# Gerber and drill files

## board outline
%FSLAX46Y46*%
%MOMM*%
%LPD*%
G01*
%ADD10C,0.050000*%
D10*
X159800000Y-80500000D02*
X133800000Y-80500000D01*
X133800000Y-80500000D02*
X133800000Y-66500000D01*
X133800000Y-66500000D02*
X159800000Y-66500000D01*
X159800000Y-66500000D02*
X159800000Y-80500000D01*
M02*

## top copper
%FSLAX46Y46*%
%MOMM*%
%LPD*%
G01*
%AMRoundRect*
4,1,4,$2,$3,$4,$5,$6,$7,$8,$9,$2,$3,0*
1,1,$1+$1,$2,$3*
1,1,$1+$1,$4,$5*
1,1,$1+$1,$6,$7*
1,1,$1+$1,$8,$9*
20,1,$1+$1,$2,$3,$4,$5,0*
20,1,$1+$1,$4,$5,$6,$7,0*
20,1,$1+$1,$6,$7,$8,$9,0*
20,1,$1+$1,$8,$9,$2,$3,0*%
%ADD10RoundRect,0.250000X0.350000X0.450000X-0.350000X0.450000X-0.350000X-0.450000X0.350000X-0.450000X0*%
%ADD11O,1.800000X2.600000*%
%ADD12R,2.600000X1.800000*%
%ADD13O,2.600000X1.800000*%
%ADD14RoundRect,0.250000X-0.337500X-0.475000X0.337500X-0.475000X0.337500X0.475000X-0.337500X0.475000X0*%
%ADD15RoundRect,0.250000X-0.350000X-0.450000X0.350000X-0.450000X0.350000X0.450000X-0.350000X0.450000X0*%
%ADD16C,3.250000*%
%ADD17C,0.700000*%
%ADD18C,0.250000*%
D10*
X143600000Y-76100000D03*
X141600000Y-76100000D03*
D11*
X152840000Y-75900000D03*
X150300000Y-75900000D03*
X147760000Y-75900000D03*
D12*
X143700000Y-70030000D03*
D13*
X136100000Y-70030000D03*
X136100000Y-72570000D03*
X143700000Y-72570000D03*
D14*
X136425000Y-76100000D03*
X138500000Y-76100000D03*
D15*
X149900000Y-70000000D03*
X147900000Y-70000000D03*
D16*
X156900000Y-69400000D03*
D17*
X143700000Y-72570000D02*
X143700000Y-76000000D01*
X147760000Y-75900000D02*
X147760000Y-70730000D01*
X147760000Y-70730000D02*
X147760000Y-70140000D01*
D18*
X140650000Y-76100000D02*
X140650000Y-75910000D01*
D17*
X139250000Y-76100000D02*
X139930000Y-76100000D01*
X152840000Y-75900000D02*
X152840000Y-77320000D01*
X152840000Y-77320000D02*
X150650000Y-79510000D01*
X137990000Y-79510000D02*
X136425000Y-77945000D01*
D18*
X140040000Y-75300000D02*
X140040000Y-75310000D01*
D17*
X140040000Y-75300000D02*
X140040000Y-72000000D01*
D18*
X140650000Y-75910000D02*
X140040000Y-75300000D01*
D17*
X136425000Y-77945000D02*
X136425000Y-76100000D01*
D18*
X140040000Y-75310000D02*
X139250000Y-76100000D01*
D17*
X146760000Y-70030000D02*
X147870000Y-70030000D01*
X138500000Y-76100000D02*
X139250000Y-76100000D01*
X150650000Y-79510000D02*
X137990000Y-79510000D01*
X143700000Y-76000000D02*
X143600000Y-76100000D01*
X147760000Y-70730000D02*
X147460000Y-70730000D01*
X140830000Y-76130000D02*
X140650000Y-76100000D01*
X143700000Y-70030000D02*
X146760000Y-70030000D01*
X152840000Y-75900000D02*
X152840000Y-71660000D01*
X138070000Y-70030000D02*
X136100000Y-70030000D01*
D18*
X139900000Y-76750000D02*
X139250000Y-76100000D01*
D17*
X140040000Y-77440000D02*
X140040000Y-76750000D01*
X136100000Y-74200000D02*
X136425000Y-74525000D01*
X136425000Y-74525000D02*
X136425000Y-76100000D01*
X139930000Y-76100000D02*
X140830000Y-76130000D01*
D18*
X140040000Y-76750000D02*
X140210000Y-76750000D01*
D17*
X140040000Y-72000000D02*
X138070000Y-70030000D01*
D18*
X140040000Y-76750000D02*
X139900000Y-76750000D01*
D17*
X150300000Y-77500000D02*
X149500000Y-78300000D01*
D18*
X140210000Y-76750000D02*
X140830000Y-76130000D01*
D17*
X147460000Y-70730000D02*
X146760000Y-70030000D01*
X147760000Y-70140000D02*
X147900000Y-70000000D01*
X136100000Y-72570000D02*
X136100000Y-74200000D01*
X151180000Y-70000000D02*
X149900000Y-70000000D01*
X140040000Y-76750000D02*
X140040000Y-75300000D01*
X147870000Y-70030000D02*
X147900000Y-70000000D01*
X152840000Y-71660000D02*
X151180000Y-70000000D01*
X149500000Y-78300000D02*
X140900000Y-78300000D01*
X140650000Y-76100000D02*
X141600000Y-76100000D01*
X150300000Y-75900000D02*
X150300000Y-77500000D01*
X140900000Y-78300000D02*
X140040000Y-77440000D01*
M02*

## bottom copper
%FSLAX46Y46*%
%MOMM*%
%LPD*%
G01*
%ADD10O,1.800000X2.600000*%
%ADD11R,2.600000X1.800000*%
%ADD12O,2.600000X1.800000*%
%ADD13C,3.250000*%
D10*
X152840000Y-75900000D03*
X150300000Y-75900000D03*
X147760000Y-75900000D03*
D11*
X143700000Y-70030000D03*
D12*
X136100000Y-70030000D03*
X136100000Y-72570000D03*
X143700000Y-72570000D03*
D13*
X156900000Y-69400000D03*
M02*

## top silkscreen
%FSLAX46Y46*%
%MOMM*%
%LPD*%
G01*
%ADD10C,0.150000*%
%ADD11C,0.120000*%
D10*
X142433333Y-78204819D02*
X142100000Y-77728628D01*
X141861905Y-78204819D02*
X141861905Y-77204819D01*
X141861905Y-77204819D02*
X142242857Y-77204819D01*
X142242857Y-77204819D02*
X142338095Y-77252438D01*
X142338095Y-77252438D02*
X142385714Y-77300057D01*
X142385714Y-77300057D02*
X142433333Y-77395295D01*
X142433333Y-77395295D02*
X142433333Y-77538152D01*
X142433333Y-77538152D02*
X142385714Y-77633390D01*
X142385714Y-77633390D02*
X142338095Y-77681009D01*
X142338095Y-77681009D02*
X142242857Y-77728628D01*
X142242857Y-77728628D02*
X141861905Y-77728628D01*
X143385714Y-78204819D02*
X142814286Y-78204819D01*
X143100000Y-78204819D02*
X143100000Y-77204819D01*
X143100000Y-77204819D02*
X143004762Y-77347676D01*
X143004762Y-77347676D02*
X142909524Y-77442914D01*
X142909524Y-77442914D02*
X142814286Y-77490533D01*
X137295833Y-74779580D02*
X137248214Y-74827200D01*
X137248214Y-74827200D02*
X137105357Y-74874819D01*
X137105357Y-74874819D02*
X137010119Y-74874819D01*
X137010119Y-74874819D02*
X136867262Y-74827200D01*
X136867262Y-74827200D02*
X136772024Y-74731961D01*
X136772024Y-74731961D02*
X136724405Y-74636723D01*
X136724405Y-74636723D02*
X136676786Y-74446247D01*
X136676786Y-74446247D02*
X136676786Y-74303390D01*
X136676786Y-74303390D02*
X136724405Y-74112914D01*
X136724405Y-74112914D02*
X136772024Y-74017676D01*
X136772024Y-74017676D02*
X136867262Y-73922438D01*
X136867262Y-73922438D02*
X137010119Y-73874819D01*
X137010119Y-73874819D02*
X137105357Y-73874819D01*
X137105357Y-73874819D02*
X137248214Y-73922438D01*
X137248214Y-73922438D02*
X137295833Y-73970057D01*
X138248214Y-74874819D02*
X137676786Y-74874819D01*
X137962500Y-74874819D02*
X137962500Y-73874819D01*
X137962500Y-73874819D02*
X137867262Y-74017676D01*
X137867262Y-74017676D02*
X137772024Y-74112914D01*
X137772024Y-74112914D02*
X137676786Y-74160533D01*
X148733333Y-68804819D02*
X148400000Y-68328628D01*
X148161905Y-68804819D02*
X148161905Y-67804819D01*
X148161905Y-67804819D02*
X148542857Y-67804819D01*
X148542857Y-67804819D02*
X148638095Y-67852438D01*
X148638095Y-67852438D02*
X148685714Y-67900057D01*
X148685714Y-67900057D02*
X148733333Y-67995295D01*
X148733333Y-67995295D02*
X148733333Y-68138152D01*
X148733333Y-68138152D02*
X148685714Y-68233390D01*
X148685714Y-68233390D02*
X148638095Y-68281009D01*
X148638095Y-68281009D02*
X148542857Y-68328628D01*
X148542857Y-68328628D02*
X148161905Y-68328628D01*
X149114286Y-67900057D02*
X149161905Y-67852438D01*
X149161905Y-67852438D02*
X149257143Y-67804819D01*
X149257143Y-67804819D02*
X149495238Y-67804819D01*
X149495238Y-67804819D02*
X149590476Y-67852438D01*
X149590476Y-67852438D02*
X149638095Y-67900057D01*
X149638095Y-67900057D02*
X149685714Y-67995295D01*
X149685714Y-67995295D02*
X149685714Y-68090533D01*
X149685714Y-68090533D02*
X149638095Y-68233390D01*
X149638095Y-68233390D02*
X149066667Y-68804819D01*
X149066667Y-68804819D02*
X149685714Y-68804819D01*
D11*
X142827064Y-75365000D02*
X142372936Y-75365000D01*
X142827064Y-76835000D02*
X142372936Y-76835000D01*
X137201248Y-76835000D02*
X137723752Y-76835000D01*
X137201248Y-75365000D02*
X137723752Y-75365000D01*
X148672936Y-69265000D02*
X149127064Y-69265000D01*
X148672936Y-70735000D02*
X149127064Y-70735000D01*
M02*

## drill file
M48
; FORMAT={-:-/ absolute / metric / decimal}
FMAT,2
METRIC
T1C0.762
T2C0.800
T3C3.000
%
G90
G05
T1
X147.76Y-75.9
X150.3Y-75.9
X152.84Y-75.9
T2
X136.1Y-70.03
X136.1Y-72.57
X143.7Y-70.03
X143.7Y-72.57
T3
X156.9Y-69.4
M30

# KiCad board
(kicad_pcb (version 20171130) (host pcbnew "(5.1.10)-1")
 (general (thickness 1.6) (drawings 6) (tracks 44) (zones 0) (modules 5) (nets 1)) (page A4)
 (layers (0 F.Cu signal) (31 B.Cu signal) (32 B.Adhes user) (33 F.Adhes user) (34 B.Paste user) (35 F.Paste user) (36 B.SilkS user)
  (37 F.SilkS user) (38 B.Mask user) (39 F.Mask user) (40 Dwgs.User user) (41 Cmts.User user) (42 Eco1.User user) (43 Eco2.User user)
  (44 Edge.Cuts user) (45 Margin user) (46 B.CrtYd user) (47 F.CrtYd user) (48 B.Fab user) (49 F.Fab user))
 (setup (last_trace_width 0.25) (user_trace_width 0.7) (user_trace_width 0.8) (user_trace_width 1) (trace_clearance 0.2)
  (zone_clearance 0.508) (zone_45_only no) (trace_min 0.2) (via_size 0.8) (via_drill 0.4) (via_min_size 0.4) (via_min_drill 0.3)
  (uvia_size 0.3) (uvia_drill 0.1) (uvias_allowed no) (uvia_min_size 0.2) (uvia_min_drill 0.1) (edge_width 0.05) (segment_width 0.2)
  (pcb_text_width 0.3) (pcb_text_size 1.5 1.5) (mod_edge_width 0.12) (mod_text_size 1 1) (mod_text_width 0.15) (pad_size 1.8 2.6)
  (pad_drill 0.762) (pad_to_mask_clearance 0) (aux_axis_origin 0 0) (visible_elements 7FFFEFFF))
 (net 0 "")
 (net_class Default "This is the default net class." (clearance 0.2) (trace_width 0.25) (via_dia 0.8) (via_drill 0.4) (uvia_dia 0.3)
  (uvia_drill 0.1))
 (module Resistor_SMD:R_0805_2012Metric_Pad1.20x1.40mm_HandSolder (layer F.Cu) (at 142.6 76.1 180)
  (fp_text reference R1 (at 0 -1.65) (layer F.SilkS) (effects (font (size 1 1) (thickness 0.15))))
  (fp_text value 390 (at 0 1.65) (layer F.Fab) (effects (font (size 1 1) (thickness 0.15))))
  (fp_line (start -0.227064 0.735) (end 0.227064 0.735) (layer F.SilkS) (width 0.12))
  (fp_line (start -0.227064 -0.735) (end 0.227064 -0.735) (layer F.SilkS) (width 0.12))
  (pad 1 smd roundrect (at -1 0 180) (size 1.2 1.4) (layers F.Cu F.Paste F.Mask) (roundrect_rratio 0.208333))
  (pad 2 smd roundrect (at 1 0 180) (size 1.2 1.4) (layers F.Cu F.Paste F.Mask) (roundrect_rratio 0.208333)))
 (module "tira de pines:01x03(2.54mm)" (layer B.Cu) (at 150.3 73.36 180)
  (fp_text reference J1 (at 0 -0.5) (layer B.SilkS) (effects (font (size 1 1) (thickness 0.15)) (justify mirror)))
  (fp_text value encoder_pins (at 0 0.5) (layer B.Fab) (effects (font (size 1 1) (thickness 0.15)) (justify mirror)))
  (pad 1 thru_hole oval (at -2.54 -2.54 180) (size 1.8 2.6) (drill 0.762) (layers *.Cu *.Mask))
  (pad 2 thru_hole oval (at 0 -2.54 180) (size 1.8 2.6) (drill 0.762) (layers *.Cu *.Mask))
  (pad 3 thru_hole oval (at 2.54 -2.54 180) (size 1.8 2.6) (drill 0.762) (layers *.Cu *.Mask)))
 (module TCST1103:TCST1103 (layer B.Cu) (at 139.9 71.3 180)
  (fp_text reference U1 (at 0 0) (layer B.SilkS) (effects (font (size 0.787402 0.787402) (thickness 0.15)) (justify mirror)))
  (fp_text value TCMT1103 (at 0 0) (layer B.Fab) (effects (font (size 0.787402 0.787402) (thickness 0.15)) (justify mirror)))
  (pad 1 thru_hole rect (at -3.8 1.27 180) (size 2.6 1.8) (drill 0.8) (layers *.Cu *.Mask) (solder_mask_margin 0.102))
  (pad 3 thru_hole oval (at 3.8 1.27 180) (size 2.6 1.8) (drill 0.8) (layers *.Cu *.Mask) (solder_mask_margin 0.102))
  (pad 4 thru_hole oval (at 3.8 -1.27 180) (size 2.6 1.8) (drill 0.8) (layers *.Cu *.Mask) (solder_mask_margin 0.102))
  (pad 2 thru_hole oval (at -3.8 -1.27 180) (size 2.6 1.8) (drill 0.8) (layers *.Cu *.Mask) (solder_mask_margin 0.102)))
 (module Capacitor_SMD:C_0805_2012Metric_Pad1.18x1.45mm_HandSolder (layer F.Cu) (at 137.4625 76.1)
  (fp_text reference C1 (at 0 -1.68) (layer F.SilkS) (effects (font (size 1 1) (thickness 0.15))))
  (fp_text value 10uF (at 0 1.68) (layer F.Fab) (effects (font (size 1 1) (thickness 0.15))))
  (fp_line (start -0.261252 0.735) (end 0.261252 0.735) (layer F.SilkS) (width 0.12))
  (fp_line (start -0.261252 -0.735) (end 0.261252 -0.735) (layer F.SilkS) (width 0.12))
  (pad 1 smd roundrect (at -1.0375 0) (size 1.175 1.45) (layers F.Cu F.Paste F.Mask) (roundrect_rratio 0.212766))
  (pad 2 smd roundrect (at 1.0375 0) (size 1.175 1.45) (layers F.Cu F.Paste F.Mask) (roundrect_rratio 0.212766)))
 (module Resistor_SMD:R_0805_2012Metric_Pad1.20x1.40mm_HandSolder (layer F.Cu) (at 148.9 70)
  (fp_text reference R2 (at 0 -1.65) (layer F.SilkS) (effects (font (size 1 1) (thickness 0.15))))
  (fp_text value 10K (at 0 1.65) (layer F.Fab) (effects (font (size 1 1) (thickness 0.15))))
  (fp_line (start -0.227064 -0.735) (end 0.227064 -0.735) (layer F.SilkS) (width 0.12))
  (fp_line (start -0.227064 0.735) (end 0.227064 0.735) (layer F.SilkS) (width 0.12))
  (pad 2 smd roundrect (at 1 0) (size 1.2 1.4) (layers F.Cu F.Paste F.Mask) (roundrect_rratio 0.208333))
  (pad 1 smd roundrect (at -1 0) (size 1.2 1.4) (layers F.Cu F.Paste F.Mask) (roundrect_rratio 0.208333)))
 (gr_line (start 159.8 80.5) (end 133.8 80.5) (layer Edge.Cuts) (width 0.05))
 (gr_line (start 133.8 80.5) (end 133.8 66.5) (layer Edge.Cuts) (width 0.05))
 (gr_line (start 133.8 66.5) (end 159.8 66.5) (layer Edge.Cuts) (width 0.05))
 (gr_line (start 159.8 66.5) (end 159.8 80.5) (layer Edge.Cuts) (width 0.05))
 (segment (start 143.7 72.57) (end 143.7 76) (width 0.7) (layer F.Cu) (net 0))
 (segment (start 147.76 75.9) (end 147.76 70.73) (width 0.7) (layer F.Cu) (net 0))
 (segment (start 147.76 70.73) (end 147.76 70.14) (width 0.7) (layer F.Cu) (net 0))
 (segment (start 140.65 76.1) (end 140.65 75.91) (width 0.25) (layer F.Cu) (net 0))
 (segment (start 139.25 76.1) (end 139.93 76.1) (width 0.7) (layer F.Cu) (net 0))
 (segment (start 152.84 75.9) (end 152.84 77.32) (width 0.7) (layer F.Cu) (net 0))
 (segment (start 152.84 77.32) (end 150.65 79.51) (width 0.7) (layer F.Cu) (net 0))
 (segment (start 137.99 79.51) (end 136.425 77.945) (width 0.7) (layer F.Cu) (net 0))
 (segment (start 140.04 75.3) (end 140.04 75.31) (width 0.25) (layer F.Cu) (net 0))
 (segment (start 140.04 75.3) (end 140.04 72) (width 0.7) (layer F.Cu) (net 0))
 (segment (start 140.65 75.91) (end 140.04 75.3) (width 0.25) (layer F.Cu) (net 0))
 (segment (start 136.425 77.945) (end 136.425 76.1) (width 0.7) (layer F.Cu) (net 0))
 (segment (start 140.04 75.31) (end 139.25 76.1) (width 0.25) (layer F.Cu) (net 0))
 (segment (start 146.76 70.03) (end 147.87 70.03) (width 0.7) (layer F.Cu) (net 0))
 (segment (start 138.5 76.1) (end 139.25 76.1) (width 0.7) (layer F.Cu) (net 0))
 (segment (start 150.65 79.51) (end 137.99 79.51) (width 0.7) (layer F.Cu) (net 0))
 (via (at 156.9 69.4) (size 3.25) (drill 3) (layers F.Cu B.Cu) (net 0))
 (segment (start 143.7 76) (end 143.6 76.1) (width 0.7) (layer F.Cu) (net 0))
 (segment (start 147.76 70.73) (end 147.46 70.73) (width 0.7) (layer F.Cu) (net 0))
 (segment (start 140.83 76.13) (end 140.65 76.1) (width 0.7) (layer F.Cu) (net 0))
 (segment (start 143.7 70.03) (end 146.76 70.03) (width 0.7) (layer F.Cu) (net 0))
 (segment (start 152.84 75.9) (end 152.84 71.66) (width 0.7) (layer F.Cu) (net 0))
 (segment (start 138.07 70.03) (end 136.1 70.03) (width 0.7) (layer F.Cu) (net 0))
 (segment (start 139.9 76.75) (end 139.25 76.1) (width 0.25) (layer F.Cu) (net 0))
 (segment (start 140.04 77.44) (end 140.04 76.75) (width 0.7) (layer F.Cu) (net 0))
 (segment (start 136.1 74.2) (end 136.425 74.525) (width 0.7) (layer F.Cu) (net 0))
 (segment (start 136.425 74.525) (end 136.425 76.1) (width 0.7) (layer F.Cu) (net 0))
 (segment (start 139.93 76.1) (end 140.83 76.13) (width 0.7) (layer F.Cu) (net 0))
 (segment (start 140.04 76.75) (end 140.21 76.75) (width 0.25) (layer F.Cu) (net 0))
 (segment (start 140.04 72) (end 138.07 70.03) (width 0.7) (layer F.Cu) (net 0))
 (segment (start 140.04 76.75) (end 139.9 76.75) (width 0.25) (layer F.Cu) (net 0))
 (segment (start 150.3 77.5) (end 149.5 78.3) (width 0.7) (layer F.Cu) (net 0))
 (segment (start 140.21 76.75) (end 140.83 76.13) (width 0.25) (layer F.Cu) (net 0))
 (segment (start 147.46 70.73) (end 146.76 70.03) (width 0.7) (layer F.Cu) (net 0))
 (segment (start 147.76 70.14) (end 147.9 70) (width 0.7) (layer F.Cu) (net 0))
 (segment (start 136.1 72.57) (end 136.1 74.2) (width 0.7) (layer F.Cu) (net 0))
 (segment (start 151.18 70) (end 149.9 70) (width 0.7) (layer F.Cu) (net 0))
 (segment (start 140.04 76.75) (end 140.04 75.3) (width 0.7) (layer F.Cu) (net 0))
 (segment (start 147.87 70.03) (end 147.9 70) (width 0.7) (layer F.Cu) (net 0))
 (segment (start 152.84 71.66) (end 151.18 70) (width 0.7) (layer F.Cu) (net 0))
 (segment (start 149.5 78.3) (end 140.9 78.3) (width 0.7) (layer F.Cu) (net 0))
 (segment (start 140.65 76.1) (end 141.6 76.1) (width 0.7) (layer F.Cu) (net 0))
 (segment (start 150.3 75.9) (end 150.3 77.5) (width 0.7) (layer F.Cu) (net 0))
 (segment (start 140.9 78.3) (end 140.04 77.44) (width 0.7) (layer F.Cu) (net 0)))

